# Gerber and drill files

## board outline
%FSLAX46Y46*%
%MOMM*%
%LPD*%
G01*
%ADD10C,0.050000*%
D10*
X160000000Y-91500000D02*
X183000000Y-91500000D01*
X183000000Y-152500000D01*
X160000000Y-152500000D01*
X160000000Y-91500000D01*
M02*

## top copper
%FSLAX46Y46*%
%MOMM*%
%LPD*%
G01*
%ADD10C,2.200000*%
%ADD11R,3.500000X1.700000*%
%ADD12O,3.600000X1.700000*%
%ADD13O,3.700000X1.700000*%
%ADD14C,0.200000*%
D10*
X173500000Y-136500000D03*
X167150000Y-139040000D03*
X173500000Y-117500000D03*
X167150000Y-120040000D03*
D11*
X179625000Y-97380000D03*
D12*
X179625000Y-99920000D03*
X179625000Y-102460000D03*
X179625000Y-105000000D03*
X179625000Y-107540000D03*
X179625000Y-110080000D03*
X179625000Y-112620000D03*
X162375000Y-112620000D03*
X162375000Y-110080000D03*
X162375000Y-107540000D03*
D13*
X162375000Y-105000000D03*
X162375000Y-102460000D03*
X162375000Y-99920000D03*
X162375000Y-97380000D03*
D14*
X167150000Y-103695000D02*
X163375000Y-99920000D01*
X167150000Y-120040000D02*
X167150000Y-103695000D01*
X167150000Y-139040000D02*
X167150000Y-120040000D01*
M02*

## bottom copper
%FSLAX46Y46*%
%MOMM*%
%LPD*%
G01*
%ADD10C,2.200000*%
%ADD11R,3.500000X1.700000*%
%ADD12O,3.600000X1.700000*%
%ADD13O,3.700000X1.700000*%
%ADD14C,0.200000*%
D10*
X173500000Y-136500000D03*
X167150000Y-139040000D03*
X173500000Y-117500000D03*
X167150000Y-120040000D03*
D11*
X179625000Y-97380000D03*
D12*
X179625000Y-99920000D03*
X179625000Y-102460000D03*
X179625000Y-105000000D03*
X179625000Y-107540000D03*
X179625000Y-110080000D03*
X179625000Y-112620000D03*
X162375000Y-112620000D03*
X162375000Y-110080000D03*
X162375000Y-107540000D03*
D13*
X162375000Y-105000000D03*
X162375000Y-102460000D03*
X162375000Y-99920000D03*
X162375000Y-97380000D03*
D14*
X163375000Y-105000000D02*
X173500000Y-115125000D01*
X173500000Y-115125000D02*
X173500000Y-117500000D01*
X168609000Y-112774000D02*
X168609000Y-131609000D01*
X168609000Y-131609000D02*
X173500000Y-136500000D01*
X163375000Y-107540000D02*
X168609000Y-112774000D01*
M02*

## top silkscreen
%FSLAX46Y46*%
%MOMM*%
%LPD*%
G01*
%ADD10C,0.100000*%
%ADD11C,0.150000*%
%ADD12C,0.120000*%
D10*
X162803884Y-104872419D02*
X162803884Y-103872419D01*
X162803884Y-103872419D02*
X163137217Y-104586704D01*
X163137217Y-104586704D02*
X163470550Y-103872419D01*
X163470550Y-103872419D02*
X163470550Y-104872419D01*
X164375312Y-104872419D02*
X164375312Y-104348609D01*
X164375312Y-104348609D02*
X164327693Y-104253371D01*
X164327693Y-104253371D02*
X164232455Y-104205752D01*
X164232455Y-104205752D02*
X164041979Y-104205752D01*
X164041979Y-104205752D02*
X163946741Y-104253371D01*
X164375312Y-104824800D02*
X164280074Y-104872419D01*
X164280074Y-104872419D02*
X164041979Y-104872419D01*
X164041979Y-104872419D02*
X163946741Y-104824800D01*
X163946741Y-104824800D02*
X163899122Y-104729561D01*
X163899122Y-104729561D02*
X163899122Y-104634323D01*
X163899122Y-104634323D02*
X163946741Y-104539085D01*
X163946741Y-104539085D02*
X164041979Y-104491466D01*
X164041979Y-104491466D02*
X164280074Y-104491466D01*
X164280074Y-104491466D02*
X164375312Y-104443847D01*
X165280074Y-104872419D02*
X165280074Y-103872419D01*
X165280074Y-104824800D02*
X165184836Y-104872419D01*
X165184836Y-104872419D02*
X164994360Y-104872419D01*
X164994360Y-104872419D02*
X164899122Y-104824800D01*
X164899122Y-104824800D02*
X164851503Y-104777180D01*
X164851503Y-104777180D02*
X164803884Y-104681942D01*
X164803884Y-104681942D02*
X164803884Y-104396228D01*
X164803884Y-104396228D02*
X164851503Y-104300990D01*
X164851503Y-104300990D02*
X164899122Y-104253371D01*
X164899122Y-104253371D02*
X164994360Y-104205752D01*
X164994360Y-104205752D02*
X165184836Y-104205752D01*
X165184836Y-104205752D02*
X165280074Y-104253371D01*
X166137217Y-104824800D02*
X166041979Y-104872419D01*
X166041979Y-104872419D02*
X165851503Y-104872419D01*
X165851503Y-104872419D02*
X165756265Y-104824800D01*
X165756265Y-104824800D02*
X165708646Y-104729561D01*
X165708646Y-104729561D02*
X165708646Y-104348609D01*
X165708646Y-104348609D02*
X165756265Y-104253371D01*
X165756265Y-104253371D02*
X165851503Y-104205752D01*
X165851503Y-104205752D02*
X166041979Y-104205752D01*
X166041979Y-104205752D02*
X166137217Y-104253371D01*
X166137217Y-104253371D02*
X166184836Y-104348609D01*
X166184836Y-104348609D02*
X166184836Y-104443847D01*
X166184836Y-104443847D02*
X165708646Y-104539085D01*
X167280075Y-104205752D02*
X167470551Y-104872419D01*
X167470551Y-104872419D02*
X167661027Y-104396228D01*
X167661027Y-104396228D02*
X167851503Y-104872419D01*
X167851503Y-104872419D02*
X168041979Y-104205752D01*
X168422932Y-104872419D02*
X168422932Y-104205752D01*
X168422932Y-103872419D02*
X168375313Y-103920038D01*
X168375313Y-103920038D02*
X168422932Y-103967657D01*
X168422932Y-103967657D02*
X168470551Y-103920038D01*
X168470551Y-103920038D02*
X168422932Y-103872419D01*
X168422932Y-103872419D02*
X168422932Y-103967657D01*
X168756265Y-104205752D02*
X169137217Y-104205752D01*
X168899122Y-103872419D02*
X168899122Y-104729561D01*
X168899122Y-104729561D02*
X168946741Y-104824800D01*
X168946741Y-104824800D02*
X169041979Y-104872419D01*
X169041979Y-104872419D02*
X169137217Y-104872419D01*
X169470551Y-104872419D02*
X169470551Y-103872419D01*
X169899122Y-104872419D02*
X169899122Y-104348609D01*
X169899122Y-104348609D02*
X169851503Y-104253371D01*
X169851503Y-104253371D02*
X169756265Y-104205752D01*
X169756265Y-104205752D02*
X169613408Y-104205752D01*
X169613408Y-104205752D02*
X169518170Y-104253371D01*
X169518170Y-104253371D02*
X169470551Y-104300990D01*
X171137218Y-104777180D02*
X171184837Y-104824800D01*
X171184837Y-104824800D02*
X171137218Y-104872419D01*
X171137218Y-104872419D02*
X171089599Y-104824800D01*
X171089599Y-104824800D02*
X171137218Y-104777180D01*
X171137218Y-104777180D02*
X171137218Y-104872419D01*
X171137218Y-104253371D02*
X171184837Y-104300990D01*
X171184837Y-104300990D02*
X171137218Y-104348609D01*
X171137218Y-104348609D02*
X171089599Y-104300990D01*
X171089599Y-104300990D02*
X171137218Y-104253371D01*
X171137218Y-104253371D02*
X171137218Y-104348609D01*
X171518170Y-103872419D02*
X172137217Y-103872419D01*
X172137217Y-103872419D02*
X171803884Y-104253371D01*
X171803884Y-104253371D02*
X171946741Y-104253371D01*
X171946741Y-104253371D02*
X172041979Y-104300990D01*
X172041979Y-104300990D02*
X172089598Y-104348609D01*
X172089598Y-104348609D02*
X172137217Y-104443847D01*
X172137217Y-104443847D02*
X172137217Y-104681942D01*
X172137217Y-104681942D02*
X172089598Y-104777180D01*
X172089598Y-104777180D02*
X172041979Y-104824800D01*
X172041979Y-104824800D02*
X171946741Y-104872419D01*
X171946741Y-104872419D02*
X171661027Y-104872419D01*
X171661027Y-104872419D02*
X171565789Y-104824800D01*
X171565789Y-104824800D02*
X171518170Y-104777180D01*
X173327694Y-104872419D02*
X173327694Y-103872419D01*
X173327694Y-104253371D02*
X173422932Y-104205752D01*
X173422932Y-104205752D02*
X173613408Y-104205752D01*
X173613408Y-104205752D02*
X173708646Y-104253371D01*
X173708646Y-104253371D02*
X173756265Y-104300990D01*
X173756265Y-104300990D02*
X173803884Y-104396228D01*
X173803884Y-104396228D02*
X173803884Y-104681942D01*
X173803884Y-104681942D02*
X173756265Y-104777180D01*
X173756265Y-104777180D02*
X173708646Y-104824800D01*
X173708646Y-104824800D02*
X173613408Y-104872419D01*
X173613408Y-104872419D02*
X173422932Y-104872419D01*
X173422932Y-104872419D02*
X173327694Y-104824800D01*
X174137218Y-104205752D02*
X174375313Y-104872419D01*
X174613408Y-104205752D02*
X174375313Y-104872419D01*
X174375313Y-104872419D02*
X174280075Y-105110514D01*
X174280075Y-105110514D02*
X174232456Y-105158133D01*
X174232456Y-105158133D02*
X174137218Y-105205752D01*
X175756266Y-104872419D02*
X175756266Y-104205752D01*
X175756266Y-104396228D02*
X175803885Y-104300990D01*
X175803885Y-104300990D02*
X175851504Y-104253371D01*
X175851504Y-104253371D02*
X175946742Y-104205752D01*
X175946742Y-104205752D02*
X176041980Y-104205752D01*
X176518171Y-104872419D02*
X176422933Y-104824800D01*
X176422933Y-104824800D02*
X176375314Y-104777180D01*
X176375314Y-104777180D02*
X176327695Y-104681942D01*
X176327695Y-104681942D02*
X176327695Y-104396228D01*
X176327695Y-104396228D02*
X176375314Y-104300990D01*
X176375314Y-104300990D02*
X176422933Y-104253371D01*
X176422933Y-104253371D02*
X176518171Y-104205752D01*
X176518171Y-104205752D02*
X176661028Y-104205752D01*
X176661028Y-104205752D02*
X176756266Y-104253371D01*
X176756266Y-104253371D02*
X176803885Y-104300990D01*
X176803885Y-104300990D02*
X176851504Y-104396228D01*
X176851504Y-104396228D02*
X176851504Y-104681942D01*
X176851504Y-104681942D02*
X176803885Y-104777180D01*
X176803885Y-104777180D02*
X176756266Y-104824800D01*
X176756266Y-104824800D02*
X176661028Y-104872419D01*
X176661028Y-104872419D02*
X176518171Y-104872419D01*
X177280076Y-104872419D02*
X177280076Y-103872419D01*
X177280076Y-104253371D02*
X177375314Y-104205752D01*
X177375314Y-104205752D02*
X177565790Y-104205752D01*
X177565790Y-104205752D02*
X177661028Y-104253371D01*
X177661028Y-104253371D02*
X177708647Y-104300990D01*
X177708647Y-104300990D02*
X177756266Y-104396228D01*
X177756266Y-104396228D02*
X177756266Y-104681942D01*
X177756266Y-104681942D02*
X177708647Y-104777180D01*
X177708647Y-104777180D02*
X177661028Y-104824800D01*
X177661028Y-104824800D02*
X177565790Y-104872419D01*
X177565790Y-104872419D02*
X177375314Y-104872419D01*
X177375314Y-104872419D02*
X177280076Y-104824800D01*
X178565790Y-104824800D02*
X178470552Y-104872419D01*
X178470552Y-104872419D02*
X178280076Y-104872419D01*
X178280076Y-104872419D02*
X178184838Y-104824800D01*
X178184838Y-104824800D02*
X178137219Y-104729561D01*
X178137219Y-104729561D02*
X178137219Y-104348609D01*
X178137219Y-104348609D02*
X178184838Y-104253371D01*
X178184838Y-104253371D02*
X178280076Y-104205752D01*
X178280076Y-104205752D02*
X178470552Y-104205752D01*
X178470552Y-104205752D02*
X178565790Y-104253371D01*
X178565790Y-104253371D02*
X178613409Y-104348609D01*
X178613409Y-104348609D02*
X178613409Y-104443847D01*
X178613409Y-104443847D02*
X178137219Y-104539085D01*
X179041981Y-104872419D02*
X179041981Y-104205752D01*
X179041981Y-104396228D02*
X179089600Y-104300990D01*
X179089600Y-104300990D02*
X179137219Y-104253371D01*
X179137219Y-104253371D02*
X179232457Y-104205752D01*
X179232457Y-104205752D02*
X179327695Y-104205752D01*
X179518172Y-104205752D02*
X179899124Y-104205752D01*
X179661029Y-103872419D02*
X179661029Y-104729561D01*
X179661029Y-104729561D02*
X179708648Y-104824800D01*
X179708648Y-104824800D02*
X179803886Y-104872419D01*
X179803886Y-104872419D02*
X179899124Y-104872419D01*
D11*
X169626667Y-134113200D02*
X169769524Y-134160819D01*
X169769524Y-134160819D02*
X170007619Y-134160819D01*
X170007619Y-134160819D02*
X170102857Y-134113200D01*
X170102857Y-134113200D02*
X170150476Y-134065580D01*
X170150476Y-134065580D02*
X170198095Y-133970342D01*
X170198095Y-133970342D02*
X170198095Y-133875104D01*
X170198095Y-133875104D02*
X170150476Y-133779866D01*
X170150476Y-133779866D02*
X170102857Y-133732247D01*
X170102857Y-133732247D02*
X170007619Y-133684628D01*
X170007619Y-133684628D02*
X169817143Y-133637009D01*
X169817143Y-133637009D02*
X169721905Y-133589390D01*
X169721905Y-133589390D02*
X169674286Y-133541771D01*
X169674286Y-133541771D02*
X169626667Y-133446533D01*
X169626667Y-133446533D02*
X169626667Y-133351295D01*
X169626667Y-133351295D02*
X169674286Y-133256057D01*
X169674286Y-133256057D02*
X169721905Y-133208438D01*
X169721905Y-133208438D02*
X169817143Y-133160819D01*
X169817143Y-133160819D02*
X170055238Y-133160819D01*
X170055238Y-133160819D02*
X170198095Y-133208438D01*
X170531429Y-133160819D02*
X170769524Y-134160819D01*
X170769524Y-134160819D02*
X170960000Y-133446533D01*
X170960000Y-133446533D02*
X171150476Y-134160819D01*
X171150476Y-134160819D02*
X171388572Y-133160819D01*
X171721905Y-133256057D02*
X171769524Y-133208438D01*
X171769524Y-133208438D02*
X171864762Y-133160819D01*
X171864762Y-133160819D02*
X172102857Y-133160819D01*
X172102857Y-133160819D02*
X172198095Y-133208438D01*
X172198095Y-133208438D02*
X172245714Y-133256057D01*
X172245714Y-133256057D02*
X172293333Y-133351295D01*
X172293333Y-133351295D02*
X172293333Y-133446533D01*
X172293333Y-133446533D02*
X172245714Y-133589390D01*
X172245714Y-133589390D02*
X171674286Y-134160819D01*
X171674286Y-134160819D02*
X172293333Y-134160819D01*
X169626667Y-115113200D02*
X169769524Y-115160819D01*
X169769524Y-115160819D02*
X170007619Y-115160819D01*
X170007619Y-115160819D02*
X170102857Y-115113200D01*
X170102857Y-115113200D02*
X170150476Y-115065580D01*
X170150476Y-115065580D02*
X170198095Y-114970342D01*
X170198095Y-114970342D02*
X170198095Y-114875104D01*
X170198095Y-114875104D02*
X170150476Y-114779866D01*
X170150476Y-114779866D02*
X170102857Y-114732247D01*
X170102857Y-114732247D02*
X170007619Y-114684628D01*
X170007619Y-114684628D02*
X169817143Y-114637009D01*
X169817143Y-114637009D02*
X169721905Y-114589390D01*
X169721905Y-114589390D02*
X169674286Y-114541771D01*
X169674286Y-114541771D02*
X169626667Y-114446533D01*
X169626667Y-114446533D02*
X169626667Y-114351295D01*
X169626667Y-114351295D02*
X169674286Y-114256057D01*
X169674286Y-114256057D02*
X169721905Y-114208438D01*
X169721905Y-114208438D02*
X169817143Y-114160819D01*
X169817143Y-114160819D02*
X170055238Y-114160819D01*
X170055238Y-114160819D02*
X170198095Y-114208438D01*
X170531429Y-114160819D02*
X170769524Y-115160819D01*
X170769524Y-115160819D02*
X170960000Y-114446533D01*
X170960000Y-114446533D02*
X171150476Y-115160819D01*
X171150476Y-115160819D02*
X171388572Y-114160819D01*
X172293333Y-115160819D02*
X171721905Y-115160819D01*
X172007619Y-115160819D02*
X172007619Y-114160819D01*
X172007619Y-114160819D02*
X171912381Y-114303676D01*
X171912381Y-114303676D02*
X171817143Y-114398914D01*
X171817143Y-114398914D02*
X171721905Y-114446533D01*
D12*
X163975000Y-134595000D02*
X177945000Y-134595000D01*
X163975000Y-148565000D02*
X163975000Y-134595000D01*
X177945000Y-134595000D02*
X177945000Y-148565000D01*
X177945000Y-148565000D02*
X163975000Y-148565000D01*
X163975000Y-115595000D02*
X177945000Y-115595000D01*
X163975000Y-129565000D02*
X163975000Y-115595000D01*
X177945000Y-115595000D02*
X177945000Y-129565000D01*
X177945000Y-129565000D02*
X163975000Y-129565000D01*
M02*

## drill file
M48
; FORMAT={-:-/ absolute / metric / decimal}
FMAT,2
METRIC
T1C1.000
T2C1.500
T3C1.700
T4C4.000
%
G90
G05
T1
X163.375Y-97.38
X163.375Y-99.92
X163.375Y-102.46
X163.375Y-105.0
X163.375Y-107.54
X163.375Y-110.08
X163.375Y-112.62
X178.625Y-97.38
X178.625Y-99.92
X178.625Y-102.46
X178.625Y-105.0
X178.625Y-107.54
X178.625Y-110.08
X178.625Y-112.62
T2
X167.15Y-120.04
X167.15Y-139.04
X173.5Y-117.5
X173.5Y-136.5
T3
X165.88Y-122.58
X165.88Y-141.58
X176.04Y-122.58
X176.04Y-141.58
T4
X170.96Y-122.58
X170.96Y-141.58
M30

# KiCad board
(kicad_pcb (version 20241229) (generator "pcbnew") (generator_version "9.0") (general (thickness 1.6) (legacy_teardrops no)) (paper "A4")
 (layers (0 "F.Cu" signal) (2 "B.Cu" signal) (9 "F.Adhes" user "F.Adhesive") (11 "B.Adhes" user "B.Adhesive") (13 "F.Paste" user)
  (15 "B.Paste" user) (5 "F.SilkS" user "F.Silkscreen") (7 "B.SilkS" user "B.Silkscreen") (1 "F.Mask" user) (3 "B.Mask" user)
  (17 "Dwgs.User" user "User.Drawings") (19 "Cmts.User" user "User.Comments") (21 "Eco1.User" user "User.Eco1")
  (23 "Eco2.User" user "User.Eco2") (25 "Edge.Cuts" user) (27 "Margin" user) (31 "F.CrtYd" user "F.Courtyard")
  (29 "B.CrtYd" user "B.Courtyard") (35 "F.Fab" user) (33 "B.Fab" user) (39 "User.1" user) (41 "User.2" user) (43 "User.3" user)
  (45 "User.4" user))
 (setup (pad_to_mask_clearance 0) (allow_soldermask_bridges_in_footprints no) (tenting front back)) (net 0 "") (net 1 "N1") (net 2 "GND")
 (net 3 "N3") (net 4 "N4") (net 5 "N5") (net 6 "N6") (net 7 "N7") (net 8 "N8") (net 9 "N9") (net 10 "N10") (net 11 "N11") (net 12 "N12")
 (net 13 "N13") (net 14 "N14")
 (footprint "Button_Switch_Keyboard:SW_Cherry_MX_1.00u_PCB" (layer "F.Cu") (at 173.5 136.5)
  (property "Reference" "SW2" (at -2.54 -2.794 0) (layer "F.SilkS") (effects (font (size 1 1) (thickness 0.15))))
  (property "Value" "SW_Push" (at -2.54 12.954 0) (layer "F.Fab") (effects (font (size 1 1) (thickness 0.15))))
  (fp_line (start -9.525 -1.905) (end 4.445 -1.905) (stroke (width 0.12) (type solid)) (layer "F.SilkS"))
  (fp_line (start -9.525 12.065) (end -9.525 -1.905) (stroke (width 0.12) (type solid)) (layer "F.SilkS"))
  (fp_line (start 4.445 -1.905) (end 4.445 12.065) (stroke (width 0.12) (type solid)) (layer "F.SilkS"))
  (fp_line (start 4.445 12.065) (end -9.525 12.065) (stroke (width 0.12) (type solid)) (layer "F.SilkS"))
  (pad "" np_thru_hole circle (at -7.62 5.08) (size 1.7 1.7) (drill 1.7) (layers "*.Cu" "*.Mask"))
  (pad "" np_thru_hole circle (at -2.54 5.08) (size 4 4) (drill 4) (layers "*.Cu" "*.Mask"))
  (pad "" np_thru_hole circle (at 2.54 5.08) (size 1.7 1.7) (drill 1.7) (layers "*.Cu" "*.Mask"))
  (pad "1" thru_hole circle (at 0 0) (size 2.2 2.2) (drill 1.5) (layers "*.Cu" "*.Mask") (remove_unused_layers no) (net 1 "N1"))
  (pad "2" thru_hole circle (at -6.35 2.54) (size 2.2 2.2) (drill 1.5) (layers "*.Cu" "*.Mask") (remove_unused_layers no) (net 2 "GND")))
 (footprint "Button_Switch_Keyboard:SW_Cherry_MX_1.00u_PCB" (layer "F.Cu") (at 173.5 117.5)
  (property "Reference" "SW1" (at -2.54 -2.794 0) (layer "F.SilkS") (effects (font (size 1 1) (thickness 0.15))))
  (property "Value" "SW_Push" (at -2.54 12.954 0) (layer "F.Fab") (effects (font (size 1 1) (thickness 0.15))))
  (fp_line (start -9.525 -1.905) (end 4.445 -1.905) (stroke (width 0.12) (type solid)) (layer "F.SilkS"))
  (fp_line (start -9.525 12.065) (end -9.525 -1.905) (stroke (width 0.12) (type solid)) (layer "F.SilkS"))
  (fp_line (start 4.445 -1.905) (end 4.445 12.065) (stroke (width 0.12) (type solid)) (layer "F.SilkS"))
  (fp_line (start 4.445 12.065) (end -9.525 12.065) (stroke (width 0.12) (type solid)) (layer "F.SilkS"))
  (pad "" np_thru_hole circle (at -7.62 5.08) (size 1.7 1.7) (drill 1.7) (layers "*.Cu" "*.Mask"))
  (pad "" np_thru_hole circle (at -2.54 5.08) (size 4 4) (drill 4) (layers "*.Cu" "*.Mask"))
  (pad "" np_thru_hole circle (at 2.54 5.08) (size 1.7 1.7) (drill 1.7) (layers "*.Cu" "*.Mask"))
  (pad "1" thru_hole circle (at 0 0) (size 2.2 2.2) (drill 1.5) (layers "*.Cu" "*.Mask") (remove_unused_layers no) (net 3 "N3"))
  (pad "2" thru_hole circle (at -6.35 2.54) (size 2.2 2.2) (drill 1.5) (layers "*.Cu" "*.Mask") (remove_unused_layers no) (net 2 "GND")))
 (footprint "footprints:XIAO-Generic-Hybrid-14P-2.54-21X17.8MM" (layer "B.Cu") (at 171 105 180)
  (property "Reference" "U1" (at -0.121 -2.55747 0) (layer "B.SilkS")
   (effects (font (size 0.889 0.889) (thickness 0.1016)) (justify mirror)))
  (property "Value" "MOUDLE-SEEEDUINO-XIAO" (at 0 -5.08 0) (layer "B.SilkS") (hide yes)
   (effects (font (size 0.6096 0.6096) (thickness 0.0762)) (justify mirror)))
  (pad "1" thru_hole rect (at -7.625 7.62 180) (size 3.5 1.7) (drill 1 (offset -1 0)) (layers "*.Cu" "*.Mask") (remove_unused_layers no)
   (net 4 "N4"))
  (pad "2" thru_hole oval (at -7.625 5.08 180) (size 3.6 1.7) (drill 1 (offset -1 0)) (layers "*.Cu" "*.Mask") (remove_unused_layers no)
   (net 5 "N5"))
  (pad "3" thru_hole oval (at -7.625 2.54 180) (size 3.6 1.7) (drill 1 (offset -1 0)) (layers "*.Cu" "*.Mask") (remove_unused_layers no)
   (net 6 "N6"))
  (pad "4" thru_hole oval (at -7.625 0 180) (size 3.6 1.7) (drill 1 (offset -1 0)) (layers "*.Cu" "*.Mask") (remove_unused_layers no)
   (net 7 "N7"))
  (pad "5" thru_hole oval (at -7.625 -2.54 180) (size 3.6 1.7) (drill 1 (offset -1 0)) (layers "*.Cu" "*.Mask") (remove_unused_layers no)
   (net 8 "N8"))
  (pad "6" thru_hole oval (at -7.625 -5.08) (size 3.6 1.7) (drill 1 (offset 1 0)) (layers "*.Cu" "*.Mask") (remove_unused_layers no)
   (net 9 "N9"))
  (pad "7" thru_hole oval (at -7.625 -7.62 180) (size 3.6 1.7) (drill 1 (offset -1 0)) (layers "*.Cu" "*.Mask") (remove_unused_layers no)
   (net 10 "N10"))
  (pad "8" thru_hole oval (at 7.625 -7.62 180) (size 3.6 1.7) (drill 1 (offset 1 0)) (layers "*.Cu" "*.Mask") (remove_unused_layers no)
   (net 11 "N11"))
  (pad "9" thru_hole oval (at 7.625 -5.08 180) (size 3.6 1.7) (drill 1 (offset 1 0)) (layers "*.Cu" "*.Mask") (remove_unused_layers no)
   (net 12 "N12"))
  (pad "10" thru_hole oval (at 7.625 -2.54 180) (size 3.6 1.7) (drill 1 (offset 1 0)) (layers "*.Cu" "*.Mask") (remove_unused_layers no)
   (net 1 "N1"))
  (pad "11" thru_hole oval (at 7.625 0 180) (size 3.7 1.7) (drill 1 (offset 1 0)) (layers "*.Cu" "*.Mask") (remove_unused_layers no)
   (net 3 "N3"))
  (pad "12" thru_hole oval (at 7.625 2.54 180) (size 3.7 1.7) (drill 1 (offset 1 0)) (layers "*.Cu" "*.Mask") (remove_unused_layers no)
   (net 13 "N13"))
  (pad "13" thru_hole oval (at 7.625 5.08 180) (size 3.7 1.7) (drill 1 (offset 1 0)) (layers "*.Cu" "*.Mask") (remove_unused_layers no)
   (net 2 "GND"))
  (pad "14" thru_hole oval (at 7.625 7.62 180) (size 3.7 1.7) (drill 1 (offset 1 0)) (layers "*.Cu" "*.Mask") (remove_unused_layers no)
   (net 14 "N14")))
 (gr_rect (start 160 91.5) (end 183 152.5) (stroke (width 0.05) (type default)) (fill no) (layer "Edge.Cuts"))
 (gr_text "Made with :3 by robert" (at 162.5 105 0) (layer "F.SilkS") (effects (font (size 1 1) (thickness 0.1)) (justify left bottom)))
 (segment (start 163.375 105) (end 173.5 115.125) (width 0.2) (layer "B.Cu") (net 3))
 (segment (start 173.5 115.125) (end 173.5 117.5) (width 0.2) (layer "B.Cu") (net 3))
 (segment (start 167.15 103.695) (end 163.375 99.92) (width 0.2) (layer "F.Cu") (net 2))
 (segment (start 167.15 120.04) (end 167.15 103.695) (width 0.2) (layer "F.Cu") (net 2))
 (segment (start 167.15 139.04) (end 167.15 120.04) (width 0.2) (layer "F.Cu") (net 2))
 (segment (start 168.609 112.774) (end 168.609 131.609) (width 0.2) (layer "B.Cu") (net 1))
 (segment (start 168.609 131.609) (end 173.5 136.5) (width 0.2) (layer "B.Cu") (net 1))
 (segment (start 163.375 107.54) (end 168.609 112.774) (width 0.2) (layer "B.Cu") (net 1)))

